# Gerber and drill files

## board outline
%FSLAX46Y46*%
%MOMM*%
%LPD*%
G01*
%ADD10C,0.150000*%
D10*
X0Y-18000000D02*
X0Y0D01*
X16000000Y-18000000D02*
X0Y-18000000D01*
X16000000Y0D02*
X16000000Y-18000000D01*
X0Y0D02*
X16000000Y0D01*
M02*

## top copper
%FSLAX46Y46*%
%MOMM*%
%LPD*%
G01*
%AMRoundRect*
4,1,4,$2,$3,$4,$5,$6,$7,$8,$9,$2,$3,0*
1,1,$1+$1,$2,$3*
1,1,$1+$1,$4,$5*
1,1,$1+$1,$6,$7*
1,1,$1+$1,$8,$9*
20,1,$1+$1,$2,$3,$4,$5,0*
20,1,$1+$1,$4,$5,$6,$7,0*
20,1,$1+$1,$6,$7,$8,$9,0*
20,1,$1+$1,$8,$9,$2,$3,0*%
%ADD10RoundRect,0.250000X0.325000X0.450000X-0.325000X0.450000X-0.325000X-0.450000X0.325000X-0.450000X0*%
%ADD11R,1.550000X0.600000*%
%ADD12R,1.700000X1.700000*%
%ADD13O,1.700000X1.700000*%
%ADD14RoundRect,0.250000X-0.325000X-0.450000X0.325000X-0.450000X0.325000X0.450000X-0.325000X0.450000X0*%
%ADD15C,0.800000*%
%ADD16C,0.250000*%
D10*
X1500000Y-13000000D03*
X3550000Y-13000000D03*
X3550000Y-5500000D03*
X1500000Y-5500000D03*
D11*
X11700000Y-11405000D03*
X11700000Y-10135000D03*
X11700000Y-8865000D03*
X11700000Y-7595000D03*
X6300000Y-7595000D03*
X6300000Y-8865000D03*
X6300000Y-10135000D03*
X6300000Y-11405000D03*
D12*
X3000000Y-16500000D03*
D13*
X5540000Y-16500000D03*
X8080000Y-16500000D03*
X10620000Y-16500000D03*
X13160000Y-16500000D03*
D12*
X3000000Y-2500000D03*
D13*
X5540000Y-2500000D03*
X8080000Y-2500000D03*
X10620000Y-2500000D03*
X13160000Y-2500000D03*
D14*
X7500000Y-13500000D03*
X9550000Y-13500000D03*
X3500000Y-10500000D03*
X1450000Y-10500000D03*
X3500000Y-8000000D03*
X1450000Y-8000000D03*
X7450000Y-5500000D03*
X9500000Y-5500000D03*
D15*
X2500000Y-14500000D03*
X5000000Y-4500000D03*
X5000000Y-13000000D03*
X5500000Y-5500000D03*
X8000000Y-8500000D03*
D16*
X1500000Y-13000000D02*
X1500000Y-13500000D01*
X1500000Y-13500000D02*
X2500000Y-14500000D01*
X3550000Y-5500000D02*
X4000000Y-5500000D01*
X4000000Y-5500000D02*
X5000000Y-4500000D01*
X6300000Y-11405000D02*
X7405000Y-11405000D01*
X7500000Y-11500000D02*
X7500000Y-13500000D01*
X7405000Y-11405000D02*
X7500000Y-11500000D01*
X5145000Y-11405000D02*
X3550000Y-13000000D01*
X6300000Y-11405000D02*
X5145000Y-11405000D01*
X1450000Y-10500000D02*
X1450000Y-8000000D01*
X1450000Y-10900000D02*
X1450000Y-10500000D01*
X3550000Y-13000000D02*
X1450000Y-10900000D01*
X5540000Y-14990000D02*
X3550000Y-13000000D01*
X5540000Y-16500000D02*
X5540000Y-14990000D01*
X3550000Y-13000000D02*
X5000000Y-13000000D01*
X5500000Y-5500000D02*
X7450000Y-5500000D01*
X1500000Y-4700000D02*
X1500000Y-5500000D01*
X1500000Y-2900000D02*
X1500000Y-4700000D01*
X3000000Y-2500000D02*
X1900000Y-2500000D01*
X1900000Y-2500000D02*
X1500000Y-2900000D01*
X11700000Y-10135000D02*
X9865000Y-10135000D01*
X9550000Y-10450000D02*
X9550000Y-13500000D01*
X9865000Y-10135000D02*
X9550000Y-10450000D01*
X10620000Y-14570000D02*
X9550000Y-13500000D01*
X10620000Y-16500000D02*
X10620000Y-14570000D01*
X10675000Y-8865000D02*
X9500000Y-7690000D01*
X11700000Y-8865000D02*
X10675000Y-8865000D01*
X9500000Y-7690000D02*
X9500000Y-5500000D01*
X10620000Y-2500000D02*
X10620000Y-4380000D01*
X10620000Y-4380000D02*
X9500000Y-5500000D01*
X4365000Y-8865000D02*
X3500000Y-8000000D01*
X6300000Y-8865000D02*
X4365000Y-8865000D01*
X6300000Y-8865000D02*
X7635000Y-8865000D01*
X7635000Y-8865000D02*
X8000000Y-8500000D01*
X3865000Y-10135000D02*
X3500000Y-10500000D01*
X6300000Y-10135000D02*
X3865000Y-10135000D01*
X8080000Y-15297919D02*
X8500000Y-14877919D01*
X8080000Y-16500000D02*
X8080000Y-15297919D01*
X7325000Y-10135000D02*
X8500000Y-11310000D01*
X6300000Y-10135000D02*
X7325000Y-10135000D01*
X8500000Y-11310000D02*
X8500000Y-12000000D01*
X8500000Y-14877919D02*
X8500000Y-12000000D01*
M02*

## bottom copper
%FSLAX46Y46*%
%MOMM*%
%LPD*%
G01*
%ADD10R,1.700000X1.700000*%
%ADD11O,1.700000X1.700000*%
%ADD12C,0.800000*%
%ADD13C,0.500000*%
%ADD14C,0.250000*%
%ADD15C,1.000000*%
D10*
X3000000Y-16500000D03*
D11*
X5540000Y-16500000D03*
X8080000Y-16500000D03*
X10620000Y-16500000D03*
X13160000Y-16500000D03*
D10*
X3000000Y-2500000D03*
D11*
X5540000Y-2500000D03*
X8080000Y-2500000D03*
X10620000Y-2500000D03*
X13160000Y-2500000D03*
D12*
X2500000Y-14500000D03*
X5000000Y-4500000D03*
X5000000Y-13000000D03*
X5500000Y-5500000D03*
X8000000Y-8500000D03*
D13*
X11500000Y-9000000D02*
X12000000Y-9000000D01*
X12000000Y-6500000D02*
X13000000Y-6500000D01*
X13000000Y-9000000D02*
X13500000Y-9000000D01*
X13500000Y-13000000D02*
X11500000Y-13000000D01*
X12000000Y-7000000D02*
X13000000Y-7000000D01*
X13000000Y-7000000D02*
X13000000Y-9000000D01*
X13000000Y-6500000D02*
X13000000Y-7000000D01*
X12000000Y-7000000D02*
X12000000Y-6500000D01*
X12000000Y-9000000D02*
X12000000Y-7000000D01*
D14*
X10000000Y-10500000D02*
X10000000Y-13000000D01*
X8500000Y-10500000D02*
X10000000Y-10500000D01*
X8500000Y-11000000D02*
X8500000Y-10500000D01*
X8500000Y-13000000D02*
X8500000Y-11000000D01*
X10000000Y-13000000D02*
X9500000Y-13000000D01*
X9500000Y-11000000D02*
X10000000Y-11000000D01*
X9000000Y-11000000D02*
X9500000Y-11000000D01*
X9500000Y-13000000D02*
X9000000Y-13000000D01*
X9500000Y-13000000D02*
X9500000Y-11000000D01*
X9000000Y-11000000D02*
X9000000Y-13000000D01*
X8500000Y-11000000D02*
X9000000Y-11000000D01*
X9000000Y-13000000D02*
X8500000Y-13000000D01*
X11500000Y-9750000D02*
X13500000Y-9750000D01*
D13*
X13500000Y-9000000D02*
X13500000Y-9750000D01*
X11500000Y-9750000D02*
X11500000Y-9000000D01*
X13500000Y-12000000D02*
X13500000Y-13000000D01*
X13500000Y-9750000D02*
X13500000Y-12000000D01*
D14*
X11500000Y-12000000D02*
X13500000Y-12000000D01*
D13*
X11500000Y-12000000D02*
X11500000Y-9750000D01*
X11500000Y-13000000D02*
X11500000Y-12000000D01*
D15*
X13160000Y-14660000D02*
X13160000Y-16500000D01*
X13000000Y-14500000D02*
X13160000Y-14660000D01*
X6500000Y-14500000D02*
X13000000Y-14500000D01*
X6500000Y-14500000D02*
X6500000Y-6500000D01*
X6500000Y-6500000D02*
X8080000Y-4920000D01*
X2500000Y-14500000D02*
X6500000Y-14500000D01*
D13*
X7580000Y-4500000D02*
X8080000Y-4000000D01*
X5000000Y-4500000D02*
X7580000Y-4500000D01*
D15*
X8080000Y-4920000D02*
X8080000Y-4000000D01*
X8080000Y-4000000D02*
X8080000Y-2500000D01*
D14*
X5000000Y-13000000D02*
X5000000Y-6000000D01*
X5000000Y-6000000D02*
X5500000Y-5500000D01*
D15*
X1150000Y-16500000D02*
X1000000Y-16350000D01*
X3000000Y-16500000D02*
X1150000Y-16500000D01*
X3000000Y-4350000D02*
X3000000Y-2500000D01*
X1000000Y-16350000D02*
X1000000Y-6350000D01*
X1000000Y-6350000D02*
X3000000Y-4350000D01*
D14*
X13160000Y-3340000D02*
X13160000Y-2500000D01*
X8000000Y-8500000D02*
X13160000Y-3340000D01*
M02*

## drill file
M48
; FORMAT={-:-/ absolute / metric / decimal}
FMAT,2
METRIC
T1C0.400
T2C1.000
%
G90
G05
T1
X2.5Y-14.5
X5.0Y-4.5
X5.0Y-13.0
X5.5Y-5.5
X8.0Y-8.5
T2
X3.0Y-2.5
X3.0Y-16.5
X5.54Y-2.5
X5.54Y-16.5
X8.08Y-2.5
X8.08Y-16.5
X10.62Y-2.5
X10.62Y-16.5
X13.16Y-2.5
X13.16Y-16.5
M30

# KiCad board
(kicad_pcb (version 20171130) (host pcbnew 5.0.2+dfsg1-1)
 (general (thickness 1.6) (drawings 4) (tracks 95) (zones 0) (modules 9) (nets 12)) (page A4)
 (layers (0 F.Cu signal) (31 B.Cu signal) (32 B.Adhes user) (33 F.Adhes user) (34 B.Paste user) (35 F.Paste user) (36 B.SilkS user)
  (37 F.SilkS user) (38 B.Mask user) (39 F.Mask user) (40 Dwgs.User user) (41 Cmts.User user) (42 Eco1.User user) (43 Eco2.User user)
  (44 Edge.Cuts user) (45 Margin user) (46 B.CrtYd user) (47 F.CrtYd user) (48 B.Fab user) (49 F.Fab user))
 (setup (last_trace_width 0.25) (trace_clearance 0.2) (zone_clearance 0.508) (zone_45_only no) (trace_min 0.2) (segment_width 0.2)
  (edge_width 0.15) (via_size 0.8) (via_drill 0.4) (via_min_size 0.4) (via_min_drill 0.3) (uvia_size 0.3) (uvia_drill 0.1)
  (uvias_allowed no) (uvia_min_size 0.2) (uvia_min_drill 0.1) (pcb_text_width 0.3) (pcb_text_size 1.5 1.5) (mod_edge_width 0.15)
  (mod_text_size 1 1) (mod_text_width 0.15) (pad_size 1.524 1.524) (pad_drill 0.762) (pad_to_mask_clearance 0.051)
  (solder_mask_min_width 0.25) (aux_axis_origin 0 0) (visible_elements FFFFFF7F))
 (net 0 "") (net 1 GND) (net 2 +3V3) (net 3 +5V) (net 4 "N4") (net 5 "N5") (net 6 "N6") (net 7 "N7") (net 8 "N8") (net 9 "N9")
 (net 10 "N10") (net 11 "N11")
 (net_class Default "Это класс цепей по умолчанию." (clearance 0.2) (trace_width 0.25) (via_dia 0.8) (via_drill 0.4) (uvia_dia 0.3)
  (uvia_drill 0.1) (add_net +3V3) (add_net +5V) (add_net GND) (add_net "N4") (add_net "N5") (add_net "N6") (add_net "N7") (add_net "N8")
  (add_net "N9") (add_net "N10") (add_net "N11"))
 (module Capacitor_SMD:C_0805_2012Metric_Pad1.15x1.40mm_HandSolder (layer F.Cu) (at 2.525 13 180)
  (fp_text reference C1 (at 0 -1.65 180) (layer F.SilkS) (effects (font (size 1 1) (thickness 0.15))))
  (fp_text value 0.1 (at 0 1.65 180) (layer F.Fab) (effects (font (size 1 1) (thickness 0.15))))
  (pad 2 smd roundrect (at 1.025 0 180) (size 1.15 1.4) (layers F.Cu F.Paste F.Mask) (roundrect_rratio 0.217391) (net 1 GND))
  (pad 1 smd roundrect (at -1.025 0 180) (size 1.15 1.4) (layers F.Cu F.Paste F.Mask) (roundrect_rratio 0.217391) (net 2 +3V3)))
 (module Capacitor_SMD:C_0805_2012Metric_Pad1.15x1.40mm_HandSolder (layer F.Cu) (at 2.525 5.5 180)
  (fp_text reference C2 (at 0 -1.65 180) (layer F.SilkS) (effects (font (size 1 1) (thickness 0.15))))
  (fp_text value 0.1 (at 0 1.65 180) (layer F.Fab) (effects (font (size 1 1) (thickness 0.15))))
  (pad 1 smd roundrect (at -1.025 0 180) (size 1.15 1.4) (layers F.Cu F.Paste F.Mask) (roundrect_rratio 0.217391) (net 1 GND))
  (pad 2 smd roundrect (at 1.025 0 180) (size 1.15 1.4) (layers F.Cu F.Paste F.Mask) (roundrect_rratio 0.217391) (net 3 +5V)))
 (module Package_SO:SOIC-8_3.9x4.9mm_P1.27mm (layer F.Cu) (at 9 9.5 180)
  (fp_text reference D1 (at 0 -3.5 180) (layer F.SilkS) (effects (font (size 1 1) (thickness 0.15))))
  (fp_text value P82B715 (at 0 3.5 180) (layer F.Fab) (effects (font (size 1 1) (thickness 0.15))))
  (pad 1 smd rect (at -2.7 -1.905 180) (size 1.55 0.6) (layers F.Cu F.Paste F.Mask) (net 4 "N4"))
  (pad 2 smd rect (at -2.7 -0.635 180) (size 1.55 0.6) (layers F.Cu F.Paste F.Mask) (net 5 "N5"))
  (pad 3 smd rect (at -2.7 0.635 180) (size 1.55 0.6) (layers F.Cu F.Paste F.Mask) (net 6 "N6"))
  (pad 4 smd rect (at -2.7 1.905 180) (size 1.55 0.6) (layers F.Cu F.Paste F.Mask) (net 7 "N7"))
  (pad 5 smd rect (at 2.7 1.905 180) (size 1.55 0.6) (layers F.Cu F.Paste F.Mask) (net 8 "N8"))
  (pad 6 smd rect (at 2.7 0.635 180) (size 1.55 0.6) (layers F.Cu F.Paste F.Mask) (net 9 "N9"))
  (pad 7 smd rect (at 2.7 -0.635 180) (size 1.55 0.6) (layers F.Cu F.Paste F.Mask) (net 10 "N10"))
  (pad 8 smd rect (at 2.7 -1.905 180) (size 1.55 0.6) (layers F.Cu F.Paste F.Mask) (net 2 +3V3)))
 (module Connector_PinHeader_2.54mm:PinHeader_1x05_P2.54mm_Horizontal (layer B.Cu) (at 3 16.5 270)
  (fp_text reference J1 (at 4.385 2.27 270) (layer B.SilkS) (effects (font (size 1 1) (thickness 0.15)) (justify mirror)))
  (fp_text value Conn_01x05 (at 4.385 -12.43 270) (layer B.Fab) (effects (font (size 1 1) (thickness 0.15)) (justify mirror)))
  (pad 1 thru_hole rect (at 0 0 270) (size 1.7 1.7) (drill 1) (layers *.Cu *.Mask) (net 3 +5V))
  (pad 2 thru_hole oval (at 0 -2.54 270) (size 1.7 1.7) (drill 1) (layers *.Cu *.Mask) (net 2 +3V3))
  (pad 3 thru_hole oval (at 0 -5.08 270) (size 1.7 1.7) (drill 1) (layers *.Cu *.Mask) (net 10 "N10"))
  (pad 4 thru_hole oval (at 0 -7.62 270) (size 1.7 1.7) (drill 1) (layers *.Cu *.Mask) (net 5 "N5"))
  (pad 5 thru_hole oval (at 0 -10.16 270) (size 1.7 1.7) (drill 1) (layers *.Cu *.Mask) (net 1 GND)))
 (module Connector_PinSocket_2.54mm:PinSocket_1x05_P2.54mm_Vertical (layer F.Cu) (at 3 2.5 90)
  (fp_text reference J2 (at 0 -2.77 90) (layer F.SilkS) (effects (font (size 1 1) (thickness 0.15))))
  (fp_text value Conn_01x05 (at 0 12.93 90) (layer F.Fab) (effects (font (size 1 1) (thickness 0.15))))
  (pad 1 thru_hole rect (at 0 0 90) (size 1.7 1.7) (drill 1) (layers *.Cu *.Mask) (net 3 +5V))
  (pad 2 thru_hole oval (at 0 2.54 90) (size 1.7 1.7) (drill 1) (layers *.Cu *.Mask) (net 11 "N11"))
  (pad 3 thru_hole oval (at 0 5.08 90) (size 1.7 1.7) (drill 1) (layers *.Cu *.Mask) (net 1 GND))
  (pad 4 thru_hole oval (at 0 7.62 90) (size 1.7 1.7) (drill 1) (layers *.Cu *.Mask) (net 6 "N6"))
  (pad 5 thru_hole oval (at 0 10.16 90) (size 1.7 1.7) (drill 1) (layers *.Cu *.Mask) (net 9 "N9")))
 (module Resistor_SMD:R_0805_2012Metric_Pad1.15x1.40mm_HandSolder (layer F.Cu) (at 8.525 13.5)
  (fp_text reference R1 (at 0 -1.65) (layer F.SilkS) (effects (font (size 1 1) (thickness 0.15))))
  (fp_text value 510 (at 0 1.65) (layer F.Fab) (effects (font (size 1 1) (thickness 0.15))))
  (pad 1 smd roundrect (at -1.025 0) (size 1.15 1.4) (layers F.Cu F.Paste F.Mask) (roundrect_rratio 0.217391) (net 2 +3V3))
  (pad 2 smd roundrect (at 1.025 0) (size 1.15 1.4) (layers F.Cu F.Paste F.Mask) (roundrect_rratio 0.217391) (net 5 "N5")))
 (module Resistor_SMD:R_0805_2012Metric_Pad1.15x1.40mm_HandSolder (layer F.Cu) (at 2.475 10.5)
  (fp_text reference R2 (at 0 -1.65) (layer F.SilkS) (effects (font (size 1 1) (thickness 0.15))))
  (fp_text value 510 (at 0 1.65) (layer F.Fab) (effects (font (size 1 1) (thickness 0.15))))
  (pad 2 smd roundrect (at 1.025 0) (size 1.15 1.4) (layers F.Cu F.Paste F.Mask) (roundrect_rratio 0.217391) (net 10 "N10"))
  (pad 1 smd roundrect (at -1.025 0) (size 1.15 1.4) (layers F.Cu F.Paste F.Mask) (roundrect_rratio 0.217391) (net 2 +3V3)))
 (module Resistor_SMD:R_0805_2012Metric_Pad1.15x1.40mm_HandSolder (layer F.Cu) (at 2.475 8)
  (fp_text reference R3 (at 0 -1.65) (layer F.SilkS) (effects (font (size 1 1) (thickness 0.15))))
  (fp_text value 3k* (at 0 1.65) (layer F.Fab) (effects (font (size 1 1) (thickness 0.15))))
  (pad 2 smd roundrect (at 1.025 0) (size 1.15 1.4) (layers F.Cu F.Paste F.Mask) (roundrect_rratio 0.217391) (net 9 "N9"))
  (pad 1 smd roundrect (at -1.025 0) (size 1.15 1.4) (layers F.Cu F.Paste F.Mask) (roundrect_rratio 0.217391) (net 2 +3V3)))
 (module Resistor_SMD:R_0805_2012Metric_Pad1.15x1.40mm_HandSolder (layer F.Cu) (at 8.475 5.5)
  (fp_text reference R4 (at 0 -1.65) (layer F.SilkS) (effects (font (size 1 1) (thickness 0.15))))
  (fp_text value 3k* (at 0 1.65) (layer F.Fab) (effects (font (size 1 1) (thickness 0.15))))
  (pad 1 smd roundrect (at -1.025 0) (size 1.15 1.4) (layers F.Cu F.Paste F.Mask) (roundrect_rratio 0.217391) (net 2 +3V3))
  (pad 2 smd roundrect (at 1.025 0) (size 1.15 1.4) (layers F.Cu F.Paste F.Mask) (roundrect_rratio 0.217391) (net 6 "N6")))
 (gr_line (start 0 18) (end 0 0) (layer Edge.Cuts) (width 0.15))
 (gr_line (start 16 18) (end 0 18) (layer Edge.Cuts) (width 0.15))
 (gr_line (start 16 0) (end 16 18) (layer Edge.Cuts) (width 0.15))
 (gr_line (start 0 0) (end 16 0) (layer Edge.Cuts) (width 0.15))
 (segment (start 11.5 9) (end 12 9) (width 0.5) (layer B.Cu) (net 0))
 (segment (start 12 6.5) (end 13 6.5) (width 0.5) (layer B.Cu) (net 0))
 (segment (start 13 9) (end 13.5 9) (width 0.5) (layer B.Cu) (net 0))
 (segment (start 13.5 13) (end 11.5 13) (width 0.5) (layer B.Cu) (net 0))
 (segment (start 12 7) (end 13 7) (width 0.5) (layer B.Cu) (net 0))
 (segment (start 13 7) (end 13 9) (width 0.5) (layer B.Cu) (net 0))
 (segment (start 13 6.5) (end 13 7) (width 0.5) (layer B.Cu) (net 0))
 (segment (start 12 7) (end 12 6.5) (width 0.5) (layer B.Cu) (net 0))
 (segment (start 12 9) (end 12 7) (width 0.5) (layer B.Cu) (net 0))
 (segment (start 10 10.5) (end 10 13) (width 0.25) (layer B.Cu) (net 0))
 (segment (start 8.5 10.5) (end 10 10.5) (width 0.25) (layer B.Cu) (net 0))
 (segment (start 8.5 11) (end 8.5 10.5) (width 0.25) (layer B.Cu) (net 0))
 (segment (start 8.5 13) (end 8.5 11) (width 0.25) (layer B.Cu) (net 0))
 (segment (start 10 13) (end 9.5 13) (width 0.25) (layer B.Cu) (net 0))
 (segment (start 9.5 11) (end 10 11) (width 0.25) (layer B.Cu) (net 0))
 (segment (start 9 11) (end 9.5 11) (width 0.25) (layer B.Cu) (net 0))
 (segment (start 9.5 13) (end 9 13) (width 0.25) (layer B.Cu) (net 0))
 (segment (start 9.5 13) (end 9.5 11) (width 0.25) (layer B.Cu) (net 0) (status 1000000))
 (segment (start 9 11) (end 9 13) (width 0.25) (layer B.Cu) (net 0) (status 1000000))
 (segment (start 8.5 11) (end 9 11) (width 0.25) (layer B.Cu) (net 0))
 (segment (start 9 13) (end 8.5 13) (width 0.25) (layer B.Cu) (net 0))
 (segment (start 11.5 9.75) (end 13.5 9.75) (width 0.25) (layer B.Cu) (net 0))
 (segment (start 13.5 9) (end 13.5 9.75) (width 0.5) (layer B.Cu) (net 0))
 (segment (start 11.5 9.75) (end 11.5 9) (width 0.5) (layer B.Cu) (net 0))
 (segment (start 13.5 12) (end 13.5 13) (width 0.5) (layer B.Cu) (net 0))
 (segment (start 13.5 9.75) (end 13.5 12) (width 0.5) (layer B.Cu) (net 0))
 (segment (start 11.5 12) (end 13.5 12) (width 0.25) (layer B.Cu) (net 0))
 (segment (start 11.5 12) (end 11.5 9.75) (width 0.5) (layer B.Cu) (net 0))
 (segment (start 11.5 13) (end 11.5 12) (width 0.5) (layer B.Cu) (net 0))
 (via (at 2.5 14.5) (size 0.8) (drill 0.4) (layers F.Cu B.Cu) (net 1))
 (segment (start 1.5 13) (end 1.5 13.5) (width 0.25) (layer F.Cu) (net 1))
 (segment (start 1.5 13.5) (end 2.5 14.5) (width 0.25) (layer F.Cu) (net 1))
 (via (at 5 4.5) (size 0.8) (drill 0.4) (layers F.Cu B.Cu) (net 1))
 (segment (start 3.55 5.5) (end 4 5.5) (width 0.25) (layer F.Cu) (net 1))
 (segment (start 4 5.5) (end 5 4.5) (width 0.25) (layer F.Cu) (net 1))
 (segment (start 13.16 14.66) (end 13.16 16.5) (width 1) (layer B.Cu) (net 1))
 (segment (start 13 14.5) (end 13.16 14.66) (width 1) (layer B.Cu) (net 1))
 (segment (start 6.5 14.5) (end 13 14.5) (width 1) (layer B.Cu) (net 1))
 (segment (start 6.5 14.5) (end 6.5 6.5) (width 1) (layer B.Cu) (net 1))
 (segment (start 6.5 6.5) (end 8.08 4.92) (width 1) (layer B.Cu) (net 1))
 (segment (start 2.5 14.5) (end 6.5 14.5) (width 1) (layer B.Cu) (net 1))
 (segment (start 7.58 4.5) (end 8.08 4) (width 0.5) (layer B.Cu) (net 1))
 (segment (start 5 4.5) (end 7.58 4.5) (width 0.5) (layer B.Cu) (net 1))
 (segment (start 8.08 4.92) (end 8.08 4) (width 1) (layer B.Cu) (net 1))
 (segment (start 8.08 4) (end 8.08 2.5) (width 1) (layer B.Cu) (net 1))
 (segment (start 6.3 11.405) (end 7.405 11.405) (width 0.25) (layer F.Cu) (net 2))
 (segment (start 7.5 11.5) (end 7.5 13.5) (width 0.25) (layer F.Cu) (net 2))
 (segment (start 7.405 11.405) (end 7.5 11.5) (width 0.25) (layer F.Cu) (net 2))
 (segment (start 5.145 11.405) (end 3.55 13) (width 0.25) (layer F.Cu) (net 2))
 (segment (start 6.3 11.405) (end 5.145 11.405) (width 0.25) (layer F.Cu) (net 2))
 (segment (start 1.45 10.5) (end 1.45 8) (width 0.25) (layer F.Cu) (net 2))
 (segment (start 1.45 10.9) (end 1.45 10.5) (width 0.25) (layer F.Cu) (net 2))
 (segment (start 3.55 13) (end 1.45 10.9) (width 0.25) (layer F.Cu) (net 2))
 (segment (start 5.54 14.99) (end 3.55 13) (width 0.25) (layer F.Cu) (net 2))
 (segment (start 5.54 16.5) (end 5.54 14.99) (width 0.25) (layer F.Cu) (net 2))
 (via (at 5 13) (size 0.8) (drill 0.4) (layers F.Cu B.Cu) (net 2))
 (segment (start 3.55 13) (end 5 13) (width 0.25) (layer F.Cu) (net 2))
 (via (at 5.5 5.5) (size 0.8) (drill 0.4) (layers F.Cu B.Cu) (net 2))
 (segment (start 5 13) (end 5 6) (width 0.25) (layer B.Cu) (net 2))
 (segment (start 5 6) (end 5.5 5.5) (width 0.25) (layer B.Cu) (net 2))
 (segment (start 5.5 5.5) (end 7.45 5.5) (width 0.25) (layer F.Cu) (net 2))
 (segment (start 1.5 4.7) (end 1.5 5.5) (width 0.25) (layer F.Cu) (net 3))
 (segment (start 1.5 2.9) (end 1.5 4.7) (width 0.25) (layer F.Cu) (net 3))
 (segment (start 3 2.5) (end 1.9 2.5) (width 0.25) (layer F.Cu) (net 3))
 (segment (start 1.9 2.5) (end 1.5 2.9) (width 0.25) (layer F.Cu) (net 3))
 (segment (start 1.15 16.5) (end 1 16.35) (width 1) (layer B.Cu) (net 3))
 (segment (start 3 16.5) (end 1.15 16.5) (width 1) (layer B.Cu) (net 3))
 (segment (start 3 4.35) (end 3 2.5) (width 1) (layer B.Cu) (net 3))
 (segment (start 1 16.35) (end 1 6.35) (width 1) (layer B.Cu) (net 3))
 (segment (start 1 6.35) (end 3 4.35) (width 1) (layer B.Cu) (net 3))
 (segment (start 11.7 10.135) (end 9.865 10.135) (width 0.25) (layer F.Cu) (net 5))
 (segment (start 9.55 10.45) (end 9.55 13.5) (width 0.25) (layer F.Cu) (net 5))
 (segment (start 9.865 10.135) (end 9.55 10.45) (width 0.25) (layer F.Cu) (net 5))
 (segment (start 10.62 14.57) (end 9.55 13.5) (width 0.25) (layer F.Cu) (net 5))
 (segment (start 10.62 16.5) (end 10.62 14.57) (width 0.25) (layer F.Cu) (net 5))
 (segment (start 10.675 8.865) (end 9.5 7.69) (width 0.25) (layer F.Cu) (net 6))
 (segment (start 11.7 8.865) (end 10.675 8.865) (width 0.25) (layer F.Cu) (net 6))
 (segment (start 9.5 7.69) (end 9.5 5.5) (width 0.25) (layer F.Cu) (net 6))
 (segment (start 10.62 2.5) (end 10.62 4.38) (width 0.25) (layer F.Cu) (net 6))
 (segment (start 10.62 4.38) (end 9.5 5.5) (width 0.25) (layer F.Cu) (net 6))
 (segment (start 4.365 8.865) (end 3.5 8) (width 0.25) (layer F.Cu) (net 9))
 (segment (start 6.3 8.865) (end 4.365 8.865) (width 0.25) (layer F.Cu) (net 9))
 (via (at 8 8.5) (size 0.8) (drill 0.4) (layers F.Cu B.Cu) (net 9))
 (segment (start 6.3 8.865) (end 7.635 8.865) (width 0.25) (layer F.Cu) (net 9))
 (segment (start 7.635 8.865) (end 8 8.5) (width 0.25) (layer F.Cu) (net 9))
 (segment (start 13.16 3.34) (end 13.16 2.5) (width 0.25) (layer B.Cu) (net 9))
 (segment (start 8 8.5) (end 13.16 3.34) (width 0.25) (layer B.Cu) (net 9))
 (segment (start 3.865 10.135) (end 3.5 10.5) (width 0.25) (layer F.Cu) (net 10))
 (segment (start 6.3 10.135) (end 3.865 10.135) (width 0.25) (layer F.Cu) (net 10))
 (segment (start 8.08 15.297919) (end 8.5 14.877919) (width 0.25) (layer F.Cu) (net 10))
 (segment (start 8.08 16.5) (end 8.08 15.297919) (width 0.25) (layer F.Cu) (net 10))
 (segment (start 7.325 10.135) (end 8.5 11.31) (width 0.25) (layer F.Cu) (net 10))
 (segment (start 6.3 10.135) (end 7.325 10.135) (width 0.25) (layer F.Cu) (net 10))
 (segment (start 8.5 11.31) (end 8.5 12) (width 0.25) (layer F.Cu) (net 10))
 (segment (start 8.5 14.877919) (end 8.5 12) (width 0.25) (layer F.Cu) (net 10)))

